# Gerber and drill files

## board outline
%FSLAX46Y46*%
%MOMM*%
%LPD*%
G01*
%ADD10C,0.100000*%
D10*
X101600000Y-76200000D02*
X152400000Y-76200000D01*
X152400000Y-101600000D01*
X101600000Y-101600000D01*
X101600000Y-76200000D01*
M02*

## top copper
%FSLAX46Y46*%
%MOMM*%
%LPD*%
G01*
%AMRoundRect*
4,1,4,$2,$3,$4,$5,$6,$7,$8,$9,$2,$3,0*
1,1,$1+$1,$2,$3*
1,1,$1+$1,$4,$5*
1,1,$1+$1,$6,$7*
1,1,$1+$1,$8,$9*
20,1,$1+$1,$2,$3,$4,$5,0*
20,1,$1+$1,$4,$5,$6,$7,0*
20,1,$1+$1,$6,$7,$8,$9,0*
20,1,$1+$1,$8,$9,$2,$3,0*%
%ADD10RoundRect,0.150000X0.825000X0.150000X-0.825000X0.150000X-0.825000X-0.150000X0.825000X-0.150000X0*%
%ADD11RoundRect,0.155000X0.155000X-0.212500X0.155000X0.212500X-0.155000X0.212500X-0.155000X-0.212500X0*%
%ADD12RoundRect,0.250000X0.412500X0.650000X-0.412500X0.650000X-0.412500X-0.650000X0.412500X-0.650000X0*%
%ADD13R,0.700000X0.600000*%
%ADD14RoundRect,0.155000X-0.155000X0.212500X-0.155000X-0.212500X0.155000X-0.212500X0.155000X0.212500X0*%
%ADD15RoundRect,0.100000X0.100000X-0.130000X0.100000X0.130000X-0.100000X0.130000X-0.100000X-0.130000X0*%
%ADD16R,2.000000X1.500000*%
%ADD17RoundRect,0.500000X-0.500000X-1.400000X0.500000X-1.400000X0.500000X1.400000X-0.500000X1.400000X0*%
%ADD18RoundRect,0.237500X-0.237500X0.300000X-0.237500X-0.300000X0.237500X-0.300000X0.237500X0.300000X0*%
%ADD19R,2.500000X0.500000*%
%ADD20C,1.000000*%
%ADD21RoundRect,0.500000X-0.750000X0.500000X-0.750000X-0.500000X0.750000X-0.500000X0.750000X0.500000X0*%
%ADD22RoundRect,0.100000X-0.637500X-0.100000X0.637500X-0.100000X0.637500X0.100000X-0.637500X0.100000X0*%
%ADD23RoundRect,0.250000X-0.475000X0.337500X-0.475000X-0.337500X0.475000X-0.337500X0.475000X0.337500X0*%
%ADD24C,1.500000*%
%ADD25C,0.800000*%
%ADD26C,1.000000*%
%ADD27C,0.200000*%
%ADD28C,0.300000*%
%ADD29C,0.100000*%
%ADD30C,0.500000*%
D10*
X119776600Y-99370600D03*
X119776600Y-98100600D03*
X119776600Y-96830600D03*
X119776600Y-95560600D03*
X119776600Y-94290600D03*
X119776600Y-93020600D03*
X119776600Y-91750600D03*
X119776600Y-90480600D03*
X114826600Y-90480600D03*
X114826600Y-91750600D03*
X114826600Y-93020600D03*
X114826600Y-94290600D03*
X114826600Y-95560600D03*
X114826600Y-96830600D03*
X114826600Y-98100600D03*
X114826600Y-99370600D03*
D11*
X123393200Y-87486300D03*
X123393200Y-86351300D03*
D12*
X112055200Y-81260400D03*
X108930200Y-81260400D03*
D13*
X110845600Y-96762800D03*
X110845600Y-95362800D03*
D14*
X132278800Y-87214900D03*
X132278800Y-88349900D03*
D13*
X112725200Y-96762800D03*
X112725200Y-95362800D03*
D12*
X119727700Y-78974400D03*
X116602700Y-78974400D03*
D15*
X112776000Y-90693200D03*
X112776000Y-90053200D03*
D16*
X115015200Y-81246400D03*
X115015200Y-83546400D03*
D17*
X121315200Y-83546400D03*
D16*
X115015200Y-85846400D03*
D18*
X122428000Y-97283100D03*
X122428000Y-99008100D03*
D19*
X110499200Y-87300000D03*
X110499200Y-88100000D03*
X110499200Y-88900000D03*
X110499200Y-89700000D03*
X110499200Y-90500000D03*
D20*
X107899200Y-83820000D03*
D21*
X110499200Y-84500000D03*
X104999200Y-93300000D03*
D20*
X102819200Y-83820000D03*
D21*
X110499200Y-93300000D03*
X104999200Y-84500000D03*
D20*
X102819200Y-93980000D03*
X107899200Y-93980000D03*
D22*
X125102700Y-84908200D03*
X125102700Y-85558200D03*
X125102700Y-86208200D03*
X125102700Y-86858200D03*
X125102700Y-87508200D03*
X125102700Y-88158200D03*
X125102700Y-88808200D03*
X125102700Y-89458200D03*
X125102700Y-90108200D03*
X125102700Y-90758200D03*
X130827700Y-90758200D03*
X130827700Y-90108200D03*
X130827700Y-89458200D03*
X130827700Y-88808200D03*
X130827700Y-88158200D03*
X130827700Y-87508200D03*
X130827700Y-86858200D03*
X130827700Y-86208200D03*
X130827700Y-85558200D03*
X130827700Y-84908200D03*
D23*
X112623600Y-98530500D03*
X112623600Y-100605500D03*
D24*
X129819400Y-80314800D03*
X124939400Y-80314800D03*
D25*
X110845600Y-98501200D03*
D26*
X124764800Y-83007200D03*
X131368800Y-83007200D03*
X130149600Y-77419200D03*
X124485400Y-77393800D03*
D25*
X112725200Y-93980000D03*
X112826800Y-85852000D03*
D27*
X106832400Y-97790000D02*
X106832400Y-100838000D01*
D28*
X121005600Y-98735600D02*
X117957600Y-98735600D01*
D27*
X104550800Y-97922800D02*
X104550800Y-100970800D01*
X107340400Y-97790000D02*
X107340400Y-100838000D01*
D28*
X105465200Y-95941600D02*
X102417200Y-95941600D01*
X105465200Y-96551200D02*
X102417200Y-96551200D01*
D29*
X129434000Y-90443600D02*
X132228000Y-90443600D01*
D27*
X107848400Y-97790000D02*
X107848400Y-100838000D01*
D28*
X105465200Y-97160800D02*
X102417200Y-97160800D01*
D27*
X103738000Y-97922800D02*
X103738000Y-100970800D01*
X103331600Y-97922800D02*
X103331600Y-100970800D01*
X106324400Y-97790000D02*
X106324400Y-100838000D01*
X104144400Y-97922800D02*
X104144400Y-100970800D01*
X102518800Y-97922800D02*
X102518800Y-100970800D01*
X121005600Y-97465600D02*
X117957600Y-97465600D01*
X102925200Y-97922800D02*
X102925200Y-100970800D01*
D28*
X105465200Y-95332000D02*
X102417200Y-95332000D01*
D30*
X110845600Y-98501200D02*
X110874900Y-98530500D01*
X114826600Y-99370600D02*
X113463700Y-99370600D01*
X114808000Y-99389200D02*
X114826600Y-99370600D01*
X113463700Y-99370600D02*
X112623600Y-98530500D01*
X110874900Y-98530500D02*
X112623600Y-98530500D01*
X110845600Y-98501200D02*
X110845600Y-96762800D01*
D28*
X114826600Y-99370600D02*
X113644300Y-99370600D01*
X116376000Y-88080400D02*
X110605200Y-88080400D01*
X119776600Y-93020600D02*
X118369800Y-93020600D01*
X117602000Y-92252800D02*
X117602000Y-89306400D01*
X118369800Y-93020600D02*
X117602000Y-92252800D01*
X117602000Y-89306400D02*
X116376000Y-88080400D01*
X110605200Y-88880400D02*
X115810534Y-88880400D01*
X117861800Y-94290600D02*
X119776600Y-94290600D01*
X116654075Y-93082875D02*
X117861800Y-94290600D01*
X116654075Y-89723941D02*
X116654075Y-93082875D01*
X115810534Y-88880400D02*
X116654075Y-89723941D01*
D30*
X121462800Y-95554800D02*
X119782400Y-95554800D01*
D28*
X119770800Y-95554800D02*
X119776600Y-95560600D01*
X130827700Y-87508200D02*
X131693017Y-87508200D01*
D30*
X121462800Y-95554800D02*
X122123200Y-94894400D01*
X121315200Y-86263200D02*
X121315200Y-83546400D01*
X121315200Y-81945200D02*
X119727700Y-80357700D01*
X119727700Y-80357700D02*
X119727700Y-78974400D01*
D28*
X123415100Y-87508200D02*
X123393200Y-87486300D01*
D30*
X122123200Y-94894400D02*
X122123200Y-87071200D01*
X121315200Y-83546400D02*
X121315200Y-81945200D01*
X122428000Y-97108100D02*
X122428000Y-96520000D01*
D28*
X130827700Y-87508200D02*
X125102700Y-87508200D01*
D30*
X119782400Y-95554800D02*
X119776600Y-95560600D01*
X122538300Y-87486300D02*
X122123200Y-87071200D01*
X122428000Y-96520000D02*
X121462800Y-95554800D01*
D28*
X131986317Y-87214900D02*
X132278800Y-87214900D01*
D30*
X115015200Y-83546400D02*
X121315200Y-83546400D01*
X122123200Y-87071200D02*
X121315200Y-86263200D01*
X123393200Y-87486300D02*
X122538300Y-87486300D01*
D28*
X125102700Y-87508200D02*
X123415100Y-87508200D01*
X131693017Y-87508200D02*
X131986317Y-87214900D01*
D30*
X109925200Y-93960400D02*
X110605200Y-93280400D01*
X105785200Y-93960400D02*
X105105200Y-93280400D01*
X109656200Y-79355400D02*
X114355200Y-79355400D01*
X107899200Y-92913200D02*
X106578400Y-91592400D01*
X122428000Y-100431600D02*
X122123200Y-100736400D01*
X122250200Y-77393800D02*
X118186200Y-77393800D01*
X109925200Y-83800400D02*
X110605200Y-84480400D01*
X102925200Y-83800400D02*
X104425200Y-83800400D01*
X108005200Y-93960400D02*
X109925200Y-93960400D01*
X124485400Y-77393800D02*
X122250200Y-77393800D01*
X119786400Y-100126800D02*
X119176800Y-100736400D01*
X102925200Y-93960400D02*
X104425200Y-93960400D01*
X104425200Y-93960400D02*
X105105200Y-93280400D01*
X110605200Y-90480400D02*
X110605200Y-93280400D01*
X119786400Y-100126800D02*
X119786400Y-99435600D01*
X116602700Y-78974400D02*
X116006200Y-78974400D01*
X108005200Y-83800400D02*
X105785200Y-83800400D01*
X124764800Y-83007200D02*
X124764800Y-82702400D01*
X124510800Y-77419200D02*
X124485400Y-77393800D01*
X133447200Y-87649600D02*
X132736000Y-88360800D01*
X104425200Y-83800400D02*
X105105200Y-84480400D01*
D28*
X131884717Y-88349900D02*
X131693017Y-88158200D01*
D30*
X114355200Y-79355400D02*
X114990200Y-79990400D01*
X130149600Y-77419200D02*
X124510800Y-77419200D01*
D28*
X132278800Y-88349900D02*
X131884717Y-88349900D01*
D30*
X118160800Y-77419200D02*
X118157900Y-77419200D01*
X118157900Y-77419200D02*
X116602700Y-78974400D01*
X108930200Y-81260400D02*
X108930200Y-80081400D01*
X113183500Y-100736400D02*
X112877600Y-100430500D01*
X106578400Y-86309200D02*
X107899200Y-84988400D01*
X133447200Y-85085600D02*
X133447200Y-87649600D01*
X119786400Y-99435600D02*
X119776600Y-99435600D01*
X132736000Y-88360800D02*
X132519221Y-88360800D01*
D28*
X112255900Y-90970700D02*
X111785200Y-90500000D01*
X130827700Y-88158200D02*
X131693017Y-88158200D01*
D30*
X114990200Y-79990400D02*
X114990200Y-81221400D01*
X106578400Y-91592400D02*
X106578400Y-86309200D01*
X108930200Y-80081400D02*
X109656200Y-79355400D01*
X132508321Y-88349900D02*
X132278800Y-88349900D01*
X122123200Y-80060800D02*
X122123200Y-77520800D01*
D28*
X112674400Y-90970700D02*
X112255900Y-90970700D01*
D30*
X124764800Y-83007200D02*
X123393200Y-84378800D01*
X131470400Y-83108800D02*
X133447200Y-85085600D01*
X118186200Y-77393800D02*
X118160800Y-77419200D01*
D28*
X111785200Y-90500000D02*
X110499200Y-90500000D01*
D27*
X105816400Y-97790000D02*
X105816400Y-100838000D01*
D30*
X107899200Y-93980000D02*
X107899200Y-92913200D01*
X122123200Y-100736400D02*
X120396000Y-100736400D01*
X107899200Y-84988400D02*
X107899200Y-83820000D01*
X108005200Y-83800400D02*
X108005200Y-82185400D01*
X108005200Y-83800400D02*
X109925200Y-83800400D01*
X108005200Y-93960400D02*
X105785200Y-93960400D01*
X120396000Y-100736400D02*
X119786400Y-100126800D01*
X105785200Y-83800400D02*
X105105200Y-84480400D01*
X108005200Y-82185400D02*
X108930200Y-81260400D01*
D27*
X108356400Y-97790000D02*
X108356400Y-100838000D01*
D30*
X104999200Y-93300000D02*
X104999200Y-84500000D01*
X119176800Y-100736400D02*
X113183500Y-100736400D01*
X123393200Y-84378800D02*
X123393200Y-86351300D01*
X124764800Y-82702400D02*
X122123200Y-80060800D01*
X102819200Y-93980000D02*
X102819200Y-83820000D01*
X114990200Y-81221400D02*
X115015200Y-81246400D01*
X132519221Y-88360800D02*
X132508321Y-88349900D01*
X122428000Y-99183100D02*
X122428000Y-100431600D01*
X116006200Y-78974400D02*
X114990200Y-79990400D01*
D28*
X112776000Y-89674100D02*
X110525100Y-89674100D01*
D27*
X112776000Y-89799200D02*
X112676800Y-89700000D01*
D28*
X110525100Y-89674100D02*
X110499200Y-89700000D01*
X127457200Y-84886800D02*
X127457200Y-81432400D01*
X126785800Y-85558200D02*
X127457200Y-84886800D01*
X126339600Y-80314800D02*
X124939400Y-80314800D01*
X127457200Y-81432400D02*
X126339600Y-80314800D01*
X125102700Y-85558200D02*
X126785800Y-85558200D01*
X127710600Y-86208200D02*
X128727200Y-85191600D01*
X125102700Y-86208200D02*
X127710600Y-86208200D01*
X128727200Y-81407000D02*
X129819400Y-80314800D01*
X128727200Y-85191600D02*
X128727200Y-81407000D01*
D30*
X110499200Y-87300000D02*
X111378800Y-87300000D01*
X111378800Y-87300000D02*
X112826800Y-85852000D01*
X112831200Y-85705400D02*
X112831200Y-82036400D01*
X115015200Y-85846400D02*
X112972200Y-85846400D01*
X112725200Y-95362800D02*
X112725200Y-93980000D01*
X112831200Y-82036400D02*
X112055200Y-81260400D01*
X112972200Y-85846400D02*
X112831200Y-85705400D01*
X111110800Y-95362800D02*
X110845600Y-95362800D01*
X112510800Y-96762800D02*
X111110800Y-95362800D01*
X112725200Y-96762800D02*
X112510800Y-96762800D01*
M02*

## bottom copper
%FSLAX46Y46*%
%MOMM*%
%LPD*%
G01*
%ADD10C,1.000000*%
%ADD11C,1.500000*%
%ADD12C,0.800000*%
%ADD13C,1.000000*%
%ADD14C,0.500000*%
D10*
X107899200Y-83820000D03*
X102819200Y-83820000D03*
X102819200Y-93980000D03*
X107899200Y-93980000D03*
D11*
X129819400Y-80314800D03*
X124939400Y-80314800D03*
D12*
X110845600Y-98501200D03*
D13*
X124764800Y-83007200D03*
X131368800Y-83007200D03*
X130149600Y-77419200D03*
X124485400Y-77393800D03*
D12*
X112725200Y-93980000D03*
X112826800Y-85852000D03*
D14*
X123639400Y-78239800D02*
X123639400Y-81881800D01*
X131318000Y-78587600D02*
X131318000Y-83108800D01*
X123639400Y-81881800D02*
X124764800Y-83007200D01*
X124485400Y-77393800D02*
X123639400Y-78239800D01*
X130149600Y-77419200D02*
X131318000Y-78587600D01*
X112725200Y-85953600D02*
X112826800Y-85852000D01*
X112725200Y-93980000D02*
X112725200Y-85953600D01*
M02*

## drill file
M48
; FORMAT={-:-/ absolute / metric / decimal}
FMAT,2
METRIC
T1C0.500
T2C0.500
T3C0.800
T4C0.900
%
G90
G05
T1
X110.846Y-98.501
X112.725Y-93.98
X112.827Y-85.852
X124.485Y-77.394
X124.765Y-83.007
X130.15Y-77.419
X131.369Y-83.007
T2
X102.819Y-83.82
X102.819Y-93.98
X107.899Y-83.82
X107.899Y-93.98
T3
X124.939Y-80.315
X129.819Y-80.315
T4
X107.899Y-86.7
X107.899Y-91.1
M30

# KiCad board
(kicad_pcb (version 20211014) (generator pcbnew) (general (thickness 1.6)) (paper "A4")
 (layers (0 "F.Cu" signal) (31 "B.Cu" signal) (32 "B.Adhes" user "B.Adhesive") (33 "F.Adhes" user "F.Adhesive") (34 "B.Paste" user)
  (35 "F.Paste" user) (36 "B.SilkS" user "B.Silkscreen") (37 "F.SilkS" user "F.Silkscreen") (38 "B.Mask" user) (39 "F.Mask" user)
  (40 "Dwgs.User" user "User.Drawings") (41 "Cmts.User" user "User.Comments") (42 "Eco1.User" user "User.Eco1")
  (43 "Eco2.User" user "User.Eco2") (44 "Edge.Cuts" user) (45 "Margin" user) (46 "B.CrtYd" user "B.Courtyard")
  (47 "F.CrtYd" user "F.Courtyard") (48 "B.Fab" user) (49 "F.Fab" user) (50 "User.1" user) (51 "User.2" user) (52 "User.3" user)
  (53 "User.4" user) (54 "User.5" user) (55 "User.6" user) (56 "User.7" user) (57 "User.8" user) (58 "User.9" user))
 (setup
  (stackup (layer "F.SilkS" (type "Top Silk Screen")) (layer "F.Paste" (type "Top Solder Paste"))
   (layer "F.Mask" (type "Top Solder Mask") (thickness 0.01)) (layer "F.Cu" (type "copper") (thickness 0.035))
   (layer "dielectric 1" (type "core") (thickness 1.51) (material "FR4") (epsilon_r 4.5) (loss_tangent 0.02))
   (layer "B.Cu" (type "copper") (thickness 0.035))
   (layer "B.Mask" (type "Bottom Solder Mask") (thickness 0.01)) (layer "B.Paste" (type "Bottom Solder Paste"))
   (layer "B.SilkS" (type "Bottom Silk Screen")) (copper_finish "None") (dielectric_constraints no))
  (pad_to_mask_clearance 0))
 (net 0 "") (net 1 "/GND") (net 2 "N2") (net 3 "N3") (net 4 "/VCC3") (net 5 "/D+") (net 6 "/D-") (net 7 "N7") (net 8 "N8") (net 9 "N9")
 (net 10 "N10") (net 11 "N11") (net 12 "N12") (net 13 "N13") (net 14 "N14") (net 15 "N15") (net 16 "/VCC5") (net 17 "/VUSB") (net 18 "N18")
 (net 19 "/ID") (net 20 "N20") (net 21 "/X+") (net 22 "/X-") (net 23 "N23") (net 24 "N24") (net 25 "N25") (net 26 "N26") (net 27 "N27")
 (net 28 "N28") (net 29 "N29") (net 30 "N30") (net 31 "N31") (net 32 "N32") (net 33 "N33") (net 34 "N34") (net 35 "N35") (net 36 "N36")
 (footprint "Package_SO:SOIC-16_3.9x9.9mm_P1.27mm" (layer "F.Cu") (at 117.3016 94.9256 180) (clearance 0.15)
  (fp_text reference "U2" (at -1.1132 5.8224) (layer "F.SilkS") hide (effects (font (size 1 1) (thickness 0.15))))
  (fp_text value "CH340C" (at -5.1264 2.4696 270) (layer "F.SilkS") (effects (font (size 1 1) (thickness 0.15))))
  (pad "1" smd roundrect (at -2.475 -4.445 180) (size 1.95 0.6) (layers "F.Cu" "F.Paste" "F.Mask") (roundrect_rratio 0.25) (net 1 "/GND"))
  (pad "2" smd roundrect (at -2.475 -3.175 180) (size 1.95 0.6) (layers "F.Cu" "F.Paste" "F.Mask") (roundrect_rratio 0.25) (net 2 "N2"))
  (pad "3" smd roundrect (at -2.475 -1.905 180) (size 1.95 0.6) (layers "F.Cu" "F.Paste" "F.Mask") (roundrect_rratio 0.25) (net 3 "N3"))
  (pad "4" smd roundrect (at -2.475 -0.635 180) (size 1.95 0.6) (layers "F.Cu" "F.Paste" "F.Mask") (roundrect_rratio 0.25) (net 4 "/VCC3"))
  (pad "5" smd roundrect (at -2.475 0.635 180) (size 1.95 0.6) (layers "F.Cu" "F.Paste" "F.Mask") (roundrect_rratio 0.25) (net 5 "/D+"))
  (pad "6" smd roundrect (at -2.475 1.905 180) (size 1.95 0.6) (layers "F.Cu" "F.Paste" "F.Mask") (roundrect_rratio 0.25) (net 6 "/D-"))
  (pad "7" smd roundrect (at -2.475 3.175 180) (size 1.95 0.6) (layers "F.Cu" "F.Paste" "F.Mask") (roundrect_rratio 0.25) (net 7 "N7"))
  (pad "8" smd roundrect (at -2.475 4.445 180) (size 1.95 0.6) (layers "F.Cu" "F.Paste" "F.Mask") (roundrect_rratio 0.25) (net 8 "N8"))
  (pad "9" smd roundrect (at 2.475 4.445 180) (size 1.95 0.6) (layers "F.Cu" "F.Paste" "F.Mask") (roundrect_rratio 0.25) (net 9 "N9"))
  (pad "10" smd roundrect (at 2.475 3.175 180) (size 1.95 0.6) (layers "F.Cu" "F.Paste" "F.Mask") (roundrect_rratio 0.25) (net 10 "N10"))
  (pad "11" smd roundrect (at 2.475 1.905 180) (size 1.95 0.6) (layers "F.Cu" "F.Paste" "F.Mask") (roundrect_rratio 0.25) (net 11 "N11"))
  (pad "12" smd roundrect (at 2.475 0.635 180) (size 1.95 0.6) (layers "F.Cu" "F.Paste" "F.Mask") (roundrect_rratio 0.25) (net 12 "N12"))
  (pad "13" smd roundrect (at 2.475 -0.635 180) (size 1.95 0.6) (layers "F.Cu" "F.Paste" "F.Mask") (roundrect_rratio 0.25) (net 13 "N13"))
  (pad "14" smd roundrect (at 2.475 -1.905 180) (size 1.95 0.6) (layers "F.Cu" "F.Paste" "F.Mask") (roundrect_rratio 0.25) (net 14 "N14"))
  (pad "15" smd roundrect (at 2.475 -3.175 180) (size 1.95 0.6) (layers "F.Cu" "F.Paste" "F.Mask") (roundrect_rratio 0.25) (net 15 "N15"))
  (pad "16" smd roundrect (at 2.475 -4.445 180) (size 1.95 0.6) (layers "F.Cu" "F.Paste" "F.Mask") (roundrect_rratio 0.25) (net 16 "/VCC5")))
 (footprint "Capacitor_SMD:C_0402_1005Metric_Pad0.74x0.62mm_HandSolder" (layer "F.Cu") (at 123.3932 86.9188 90)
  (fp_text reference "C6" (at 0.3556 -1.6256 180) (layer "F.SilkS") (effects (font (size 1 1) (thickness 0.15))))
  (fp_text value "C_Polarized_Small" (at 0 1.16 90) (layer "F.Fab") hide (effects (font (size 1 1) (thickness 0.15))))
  (pad "1" smd roundrect (at -0.5675 0 90) (size 0.735 0.62) (layers "F.Cu" "F.Paste" "F.Mask") (roundrect_rratio 0.25) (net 4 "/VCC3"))
  (pad "2" smd roundrect (at 0.5675 0 90) (size 0.735 0.62) (layers "F.Cu" "F.Paste" "F.Mask") (roundrect_rratio 0.25) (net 1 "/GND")))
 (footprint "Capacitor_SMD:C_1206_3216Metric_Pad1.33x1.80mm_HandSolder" (layer "F.Cu") (at 110.4927 81.2604 180)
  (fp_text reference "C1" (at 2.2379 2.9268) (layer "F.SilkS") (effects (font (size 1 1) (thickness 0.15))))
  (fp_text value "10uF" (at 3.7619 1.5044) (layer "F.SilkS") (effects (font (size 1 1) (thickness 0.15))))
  (pad "1" smd roundrect (at -1.5625 0 180) (size 1.325 1.8) (layers "F.Cu" "F.Paste" "F.Mask") (roundrect_rratio 0.188679) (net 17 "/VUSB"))
  (pad "2" smd roundrect (at 1.5625 0 180) (size 1.325 1.8) (layers "F.Cu" "F.Paste" "F.Mask") (roundrect_rratio 0.188679) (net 1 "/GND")))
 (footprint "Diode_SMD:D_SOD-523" (layer "F.Cu") (at 110.8456 96.0628 90)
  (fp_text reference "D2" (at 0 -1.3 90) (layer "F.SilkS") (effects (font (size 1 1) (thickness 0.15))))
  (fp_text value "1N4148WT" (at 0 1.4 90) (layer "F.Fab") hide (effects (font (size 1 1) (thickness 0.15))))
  (pad "1" smd rect (at -0.7 0 270) (size 0.6 0.7) (layers "F.Cu" "F.Paste" "F.Mask") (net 16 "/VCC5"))
  (pad "2" smd rect (at 0.7 0 270) (size 0.6 0.7) (layers "F.Cu" "F.Paste" "F.Mask") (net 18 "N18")))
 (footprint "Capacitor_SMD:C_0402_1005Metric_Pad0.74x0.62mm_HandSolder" (layer "F.Cu") (at 132.2788 87.7824 -90)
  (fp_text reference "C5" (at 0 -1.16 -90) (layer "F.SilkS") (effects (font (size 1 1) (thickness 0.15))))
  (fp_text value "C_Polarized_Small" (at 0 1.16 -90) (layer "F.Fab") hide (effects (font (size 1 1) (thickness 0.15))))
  (pad "1" smd roundrect (at -0.5675 0 270) (size 0.735 0.62) (layers "F.Cu" "F.Paste" "F.Mask") (roundrect_rratio 0.25) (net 4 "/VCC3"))
  (pad "2" smd roundrect (at 0.5675 0 270) (size 0.735 0.62) (layers "F.Cu" "F.Paste" "F.Mask") (roundrect_rratio 0.25) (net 1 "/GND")))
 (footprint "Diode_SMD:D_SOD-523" (layer "F.Cu") (at 112.7252 96.0628 90)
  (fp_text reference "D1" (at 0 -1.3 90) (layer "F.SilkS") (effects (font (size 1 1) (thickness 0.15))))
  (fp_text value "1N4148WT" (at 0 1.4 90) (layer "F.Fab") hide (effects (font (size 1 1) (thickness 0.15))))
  (pad "1" smd rect (at -0.7 0 270) (size 0.6 0.7) (layers "F.Cu" "F.Paste" "F.Mask") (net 18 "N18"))
  (pad "2" smd rect (at 0.7 0 270) (size 0.6 0.7) (layers "F.Cu" "F.Paste" "F.Mask") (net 17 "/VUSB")))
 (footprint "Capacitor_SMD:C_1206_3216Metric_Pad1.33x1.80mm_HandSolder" (layer "F.Cu") (at 118.1652 78.9744 180)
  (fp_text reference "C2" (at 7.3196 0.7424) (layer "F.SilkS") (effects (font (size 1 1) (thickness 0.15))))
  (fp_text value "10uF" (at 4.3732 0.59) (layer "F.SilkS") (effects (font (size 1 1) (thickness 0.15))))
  (pad "1" smd roundrect (at -1.5625 0 180) (size 1.325 1.8) (layers "F.Cu" "F.Paste" "F.Mask") (roundrect_rratio 0.188679) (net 4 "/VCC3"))
  (pad "2" smd roundrect (at 1.5625 0 180) (size 1.325 1.8) (layers "F.Cu" "F.Paste" "F.Mask") (roundrect_rratio 0.188679) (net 1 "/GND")))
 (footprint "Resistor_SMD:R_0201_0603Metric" (layer "F.Cu") (at 112.776 90.3732 90)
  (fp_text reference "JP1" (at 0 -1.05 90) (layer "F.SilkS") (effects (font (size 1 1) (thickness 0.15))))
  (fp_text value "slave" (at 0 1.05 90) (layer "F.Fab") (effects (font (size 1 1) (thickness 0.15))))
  (pad "" smd roundrect (at -0.345 0 90) (size 0.318 0.36) (layers "F.Paste") (roundrect_rratio 0.25))
  (pad "" smd roundrect (at 0.345 0 90) (size 0.318 0.36) (layers "F.Paste") (roundrect_rratio 0.25))
  (pad "1" smd roundrect (at -0.32 0 90) (size 0.46 0.4) (layers "F.Cu" "F.Mask") (roundrect_rratio 0.25) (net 1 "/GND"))
  (pad "2" smd roundrect (at 0.32 0 90) (size 0.46 0.4) (layers "F.Cu" "F.Mask") (roundrect_rratio 0.25) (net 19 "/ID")))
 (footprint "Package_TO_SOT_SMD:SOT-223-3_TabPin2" (layer "F.Cu") (at 118.1652 83.5464)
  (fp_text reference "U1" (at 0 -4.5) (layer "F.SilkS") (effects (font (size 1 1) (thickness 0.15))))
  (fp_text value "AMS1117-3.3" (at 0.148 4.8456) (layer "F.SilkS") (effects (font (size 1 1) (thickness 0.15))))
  (pad "1" smd rect (at -3.15 -2.3) (size 2 1.5) (layers "F.Cu" "F.Paste" "F.Mask") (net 1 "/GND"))
  (pad "2" smd rect (at -3.15 0) (size 2 1.5) (layers "F.Cu" "F.Paste" "F.Mask") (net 4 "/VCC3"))
  (pad "2" smd roundrect (at 3.15 0) (size 2 3.8) (layers "F.Cu" "F.Paste" "F.Mask") (roundrect_rratio 0.25) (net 4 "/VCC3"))
  (pad "3" smd rect (at -3.15 2.3) (size 2 1.5) (layers "F.Cu" "F.Paste" "F.Mask") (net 17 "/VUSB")))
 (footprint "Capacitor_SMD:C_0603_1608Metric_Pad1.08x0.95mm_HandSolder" (layer "F.Cu") (at 122.428 98.1456 -90)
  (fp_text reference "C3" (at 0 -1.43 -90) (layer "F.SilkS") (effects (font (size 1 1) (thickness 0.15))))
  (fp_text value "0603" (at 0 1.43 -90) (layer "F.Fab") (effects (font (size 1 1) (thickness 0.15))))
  (pad "1" smd roundrect (at -0.8625 0 270) (size 1.075 0.95) (layers "F.Cu" "F.Paste" "F.Mask") (roundrect_rratio 0.25) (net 4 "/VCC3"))
  (pad "2" smd roundrect (at 0.8625 0 270) (size 1.075 0.95) (layers "F.Cu" "F.Paste" "F.Mask") (roundrect_rratio 0.25) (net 1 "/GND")))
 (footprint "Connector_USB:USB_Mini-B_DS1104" (layer "F.Cu") (at 107.8992 88.9 -90)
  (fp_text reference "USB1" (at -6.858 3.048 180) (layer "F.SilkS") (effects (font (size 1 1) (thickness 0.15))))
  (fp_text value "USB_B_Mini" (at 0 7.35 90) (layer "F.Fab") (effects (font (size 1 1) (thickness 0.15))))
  (pad "" np_thru_hole circle (at 2.2 0 270) (size 0.9 0.9) (drill 0.9) (layers *.Cu *.Mask))
  (pad "" np_thru_hole circle (at -2.2 0 270) (size 0.9 0.9) (drill 0.9) (layers *.Cu *.Mask))
  (pad "1" smd rect (at -1.6 -2.6 270) (size 0.5 2.5) (layers "F.Cu" "F.Paste" "F.Mask") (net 17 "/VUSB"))
  (pad "2" smd rect (at -0.8 -2.6 270) (size 0.5 2.5) (layers "F.Cu" "F.Paste" "F.Mask") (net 6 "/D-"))
  (pad "3" smd rect (at 0 -2.6 270) (size 0.5 2.5) (layers "F.Cu" "F.Paste" "F.Mask") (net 5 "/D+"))
  (pad "4" smd rect (at 0.8 -2.6 270) (size 0.5 2.5) (layers "F.Cu" "F.Paste" "F.Mask") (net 19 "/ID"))
  (pad "5" smd rect (at 1.6 -2.6 270) (size 0.5 2.5) (layers "F.Cu" "F.Paste" "F.Mask") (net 1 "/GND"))
  (pad "6" thru_hole circle (at -5.08 0 270) (size 1 1) (drill 0.5) (layers *.Cu *.Mask) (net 1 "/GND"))
  (pad "6" smd roundrect (at -4.4 -2.6 270) (size 2 2.5) (layers "F.Cu" "F.Paste" "F.Mask") (roundrect_rratio 0.25) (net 1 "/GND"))
  (pad "6" smd roundrect (at 4.4 2.9 270) (size 2 2.5) (layers "F.Cu" "F.Paste" "F.Mask") (roundrect_rratio 0.25) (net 1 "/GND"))
  (pad "6" thru_hole circle (at -5.08 5.08 270) (size 1 1) (drill 0.5) (layers *.Cu *.Mask) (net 1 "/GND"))
  (pad "6" smd roundrect (at 4.4 -2.6 270) (size 2 2.5) (layers "F.Cu" "F.Paste" "F.Mask") (roundrect_rratio 0.25) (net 1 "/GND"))
  (pad "6" smd roundrect (at -4.4 2.9 270) (size 2 2.5) (layers "F.Cu" "F.Paste" "F.Mask") (roundrect_rratio 0.25) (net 1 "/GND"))
  (pad "6" thru_hole circle (at 5.08 5.08 270) (size 1 1) (drill 0.5) (layers *.Cu *.Mask) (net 1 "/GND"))
  (pad "6" thru_hole circle (at 5.08 0 270) (size 1 1) (drill 0.5) (layers *.Cu *.Mask) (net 1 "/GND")))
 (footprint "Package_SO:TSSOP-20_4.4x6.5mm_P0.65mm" (layer "F.Cu") (at 127.9652 87.8332)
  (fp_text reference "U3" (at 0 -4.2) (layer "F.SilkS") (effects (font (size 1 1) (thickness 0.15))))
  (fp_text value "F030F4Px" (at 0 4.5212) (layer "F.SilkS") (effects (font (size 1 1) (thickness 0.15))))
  (pad "1" smd roundrect (at -2.8625 -2.925) (size 1.475 0.4) (layers "F.Cu" "F.Paste" "F.Mask") (roundrect_rratio 0.25) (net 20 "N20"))
  (pad "2" smd roundrect (at -2.8625 -2.275) (size 1.475 0.4) (layers "F.Cu" "F.Paste" "F.Mask") (roundrect_rratio 0.25) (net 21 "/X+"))
  (pad "3" smd roundrect (at -2.8625 -1.625) (size 1.475 0.4) (layers "F.Cu" "F.Paste" "F.Mask") (roundrect_rratio 0.25) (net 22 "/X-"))
  (pad "4" smd roundrect (at -2.8625 -0.975) (size 1.475 0.4) (layers "F.Cu" "F.Paste" "F.Mask") (roundrect_rratio 0.25) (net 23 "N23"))
  (pad "5" smd roundrect (at -2.8625 -0.325) (size 1.475 0.4) (layers "F.Cu" "F.Paste" "F.Mask") (roundrect_rratio 0.25) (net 4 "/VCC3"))
  (pad "6" smd roundrect (at -2.8625 0.325) (size 1.475 0.4) (layers "F.Cu" "F.Paste" "F.Mask") (roundrect_rratio 0.25) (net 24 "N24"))
  (pad "7" smd roundrect (at -2.8625 0.975) (size 1.475 0.4) (layers "F.Cu" "F.Paste" "F.Mask") (roundrect_rratio 0.25) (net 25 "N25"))
  (pad "8" smd roundrect (at -2.8625 1.625) (size 1.475 0.4) (layers "F.Cu" "F.Paste" "F.Mask") (roundrect_rratio 0.25) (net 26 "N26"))
  (pad "9" smd roundrect (at -2.8625 2.275) (size 1.475 0.4) (layers "F.Cu" "F.Paste" "F.Mask") (roundrect_rratio 0.25) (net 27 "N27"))
  (pad "10" smd roundrect (at -2.8625 2.925) (size 1.475 0.4) (layers "F.Cu" "F.Paste" "F.Mask") (roundrect_rratio 0.25) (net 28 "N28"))
  (pad "11" smd roundrect (at 2.8625 2.925) (size 1.475 0.4) (layers "F.Cu" "F.Paste" "F.Mask") (roundrect_rratio 0.25) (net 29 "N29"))
  (pad "12" smd roundrect (at 2.8625 2.275) (size 1.475 0.4) (layers "F.Cu" "F.Paste" "F.Mask") (roundrect_rratio 0.25) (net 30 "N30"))
  (pad "13" smd roundrect (at 2.8625 1.625) (size 1.475 0.4) (layers "F.Cu" "F.Paste" "F.Mask") (roundrect_rratio 0.25) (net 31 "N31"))
  (pad "14" smd roundrect (at 2.8625 0.975) (size 1.475 0.4) (layers "F.Cu" "F.Paste" "F.Mask") (roundrect_rratio 0.25) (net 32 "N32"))
  (pad "15" smd roundrect (at 2.8625 0.325) (size 1.475 0.4) (layers "F.Cu" "F.Paste" "F.Mask") (roundrect_rratio 0.25) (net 1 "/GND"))
  (pad "16" smd roundrect (at 2.8625 -0.325) (size 1.475 0.4) (layers "F.Cu" "F.Paste" "F.Mask") (roundrect_rratio 0.25) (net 4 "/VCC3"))
  (pad "17" smd roundrect (at 2.8625 -0.975) (size 1.475 0.4) (layers "F.Cu" "F.Paste" "F.Mask") (roundrect_rratio 0.25) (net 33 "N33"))
  (pad "18" smd roundrect (at 2.8625 -1.625) (size 1.475 0.4) (layers "F.Cu" "F.Paste" "F.Mask") (roundrect_rratio 0.25) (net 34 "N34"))
  (pad "19" smd roundrect (at 2.8625 -2.275) (size 1.475 0.4) (layers "F.Cu" "F.Paste" "F.Mask") (roundrect_rratio 0.25) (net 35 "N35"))
  (pad "20" smd roundrect (at 2.8625 -2.925) (size 1.475 0.4) (layers "F.Cu" "F.Paste" "F.Mask") (roundrect_rratio 0.25) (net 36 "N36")))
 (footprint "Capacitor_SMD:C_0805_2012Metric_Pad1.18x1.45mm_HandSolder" (layer "F.Cu") (at 112.6236 99.568 -90)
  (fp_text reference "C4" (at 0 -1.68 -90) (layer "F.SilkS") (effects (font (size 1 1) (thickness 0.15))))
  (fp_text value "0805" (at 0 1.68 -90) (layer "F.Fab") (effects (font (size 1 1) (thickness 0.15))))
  (pad "1" smd roundrect (at -1.0375 0 270) (size 1.175 1.45) (layers "F.Cu" "F.Paste" "F.Mask") (roundrect_rratio 0.212766)
   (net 16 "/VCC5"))
  (pad "2" smd roundrect (at 1.0375 0 270) (size 1.175 1.45) (layers "F.Cu" "F.Paste" "F.Mask") (roundrect_rratio 0.212766) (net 1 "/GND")))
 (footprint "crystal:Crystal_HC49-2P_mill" (layer "B.Cu") (at 129.8194 80.3148 180)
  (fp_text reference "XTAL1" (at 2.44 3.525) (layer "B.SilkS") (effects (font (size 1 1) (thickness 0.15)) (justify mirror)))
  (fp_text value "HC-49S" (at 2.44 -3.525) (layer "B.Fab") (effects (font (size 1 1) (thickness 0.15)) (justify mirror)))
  (pad "1" thru_hole circle (at 0 0 180) (size 1.5 1.5) (drill 0.8) (layers *.Cu *.Mask) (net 22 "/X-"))
  (pad "2" thru_hole circle (at 4.88 0 180) (size 1.5 1.5) (drill 0.8) (layers *.Cu *.Mask) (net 21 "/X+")))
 (gr_rect (start 101.6 76.2) (end 152.4 101.6) (layer "Edge.Cuts") (width 0.1) (fill none))
 (segment (start 106.8324 97.79) (end 106.8324 100.838) (width 0.2) (layer "F.Cu") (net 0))
 (segment (start 121.0056 98.7356) (end 117.9576 98.7356) (width 0.3) (layer "F.Cu") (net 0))
 (segment (start 104.5508 97.9228) (end 104.5508 100.9708) (width 0.2) (layer "F.Cu") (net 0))
 (segment (start 107.3404 97.79) (end 107.3404 100.838) (width 0.2) (layer "F.Cu") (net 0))
 (segment (start 105.4652 95.9416) (end 102.4172 95.9416) (width 0.3) (layer "F.Cu") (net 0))
 (segment (start 105.4652 96.5512) (end 102.4172 96.5512) (width 0.3) (layer "F.Cu") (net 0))
 (segment (start 129.434 90.4436) (end 132.228 90.4436) (width 0.1) (layer "F.Cu") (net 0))
 (segment (start 107.8484 97.79) (end 107.8484 100.838) (width 0.2) (layer "F.Cu") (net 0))
 (segment (start 105.4652 97.1608) (end 102.4172 97.1608) (width 0.3) (layer "F.Cu") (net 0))
 (segment (start 103.738 97.9228) (end 103.738 100.9708) (width 0.2) (layer "F.Cu") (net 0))
 (segment (start 103.3316 97.9228) (end 103.3316 100.9708) (width 0.2) (layer "F.Cu") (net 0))
 (segment (start 106.3244 97.79) (end 106.3244 100.838) (width 0.2) (layer "F.Cu") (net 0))
 (segment (start 104.1444 97.9228) (end 104.1444 100.9708) (width 0.2) (layer "F.Cu") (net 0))
 (segment (start 102.5188 97.9228) (end 102.5188 100.9708) (width 0.2) (layer "F.Cu") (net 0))
 (segment (start 121.0056 97.4656) (end 117.9576 97.4656) (width 0.2) (layer "F.Cu") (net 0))
 (segment (start 102.9252 97.9228) (end 102.9252 100.9708) (width 0.2) (layer "F.Cu") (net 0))
 (segment (start 105.4652 95.332) (end 102.4172 95.332) (width 0.3) (layer "F.Cu") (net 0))
 (segment (start 110.8456 98.5012) (end 110.8749 98.5305) (width 0.5) (layer "F.Cu") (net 16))
 (segment (start 114.8266 99.3706) (end 113.4637 99.3706) (width 0.5) (layer "F.Cu") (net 16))
 (segment (start 114.808 99.3892) (end 114.8266 99.3706) (width 0.5) (layer "F.Cu") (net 16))
 (segment (start 113.4637 99.3706) (end 112.6236 98.5305) (width 0.5) (layer "F.Cu") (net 16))
 (segment (start 110.8749 98.5305) (end 112.6236 98.5305) (width 0.5) (layer "F.Cu") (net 16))
 (segment (start 110.8456 98.5012) (end 110.8456 96.7628) (width 0.5) (layer "F.Cu") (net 16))
 (segment (start 114.8266 99.3706) (end 113.6443 99.3706) (width 0.3) (layer "F.Cu") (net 16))
 (via (at 110.8456 98.5012) (size 0.8) (drill 0.5) (layers "F.Cu" "B.Cu") (free) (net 16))
 (segment (start 116.376 88.0804) (end 110.6052 88.0804) (width 0.3) (layer "F.Cu") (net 6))
 (segment (start 119.7766 93.0206) (end 118.3698 93.0206) (width 0.3) (layer "F.Cu") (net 6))
 (segment (start 117.602 92.2528) (end 117.602 89.3064) (width 0.3) (layer "F.Cu") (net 6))
 (segment (start 118.3698 93.0206) (end 117.602 92.2528) (width 0.3) (layer "F.Cu") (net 6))
 (segment (start 117.602 89.3064) (end 116.376 88.0804) (width 0.3) (layer "F.Cu") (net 6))
 (segment (start 110.6052 88.8804) (end 115.810534 88.8804) (width 0.3) (layer "F.Cu") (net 5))
 (segment (start 117.8618 94.2906) (end 119.7766 94.2906) (width 0.3) (layer "F.Cu") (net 5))
 (segment (start 116.654075 93.082875) (end 117.8618 94.2906) (width 0.3) (layer "F.Cu") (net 5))
 (segment (start 116.654075 89.723941) (end 116.654075 93.082875) (width 0.3) (layer "F.Cu") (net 5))
 (segment (start 115.810534 88.8804) (end 116.654075 89.723941) (width 0.3) (layer "F.Cu") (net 5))
 (segment (start 121.4628 95.5548) (end 119.7824 95.5548) (width 0.5) (layer "F.Cu") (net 4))
 (segment (start 119.7708 95.5548) (end 119.7766 95.5606) (width 0.3) (layer "F.Cu") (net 4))
 (segment (start 130.8277 87.5082) (end 131.693017 87.5082) (width 0.3) (layer "F.Cu") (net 4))
 (segment (start 121.4628 95.5548) (end 122.1232 94.8944) (width 0.5) (layer "F.Cu") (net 4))
 (segment (start 121.3152 86.2632) (end 121.3152 83.5464) (width 0.5) (layer "F.Cu") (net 4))
 (segment (start 121.3152 81.9452) (end 119.7277 80.3577) (width 0.5) (layer "F.Cu") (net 4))
 (segment (start 119.7277 80.3577) (end 119.7277 78.9744) (width 0.5) (layer "F.Cu") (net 4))
 (segment (start 123.4151 87.5082) (end 123.3932 87.4863) (width 0.3) (layer "F.Cu") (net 4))
 (segment (start 122.1232 94.8944) (end 122.1232 87.0712) (width 0.5) (layer "F.Cu") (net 4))
 (segment (start 121.3152 83.5464) (end 121.3152 81.9452) (width 0.5) (layer "F.Cu") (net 4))
 (segment (start 122.428 97.1081) (end 122.428 96.52) (width 0.5) (layer "F.Cu") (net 4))
 (segment (start 130.8277 87.5082) (end 125.1027 87.5082) (width 0.3) (layer "F.Cu") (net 4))
 (segment (start 119.7824 95.5548) (end 119.7766 95.5606) (width 0.5) (layer "F.Cu") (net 4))
 (segment (start 122.5383 87.4863) (end 122.1232 87.0712) (width 0.5) (layer "F.Cu") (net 4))
 (segment (start 122.428 96.52) (end 121.4628 95.5548) (width 0.5) (layer "F.Cu") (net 4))
 (segment (start 131.986317 87.2149) (end 132.2788 87.2149) (width 0.3) (layer "F.Cu") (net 4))
 (segment (start 115.0152 83.5464) (end 121.3152 83.5464) (width 0.5) (layer "F.Cu") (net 4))
 (segment (start 122.1232 87.0712) (end 121.3152 86.2632) (width 0.5) (layer "F.Cu") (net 4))
 (segment (start 123.3932 87.4863) (end 122.5383 87.4863) (width 0.5) (layer "F.Cu") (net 4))
 (segment (start 125.1027 87.5082) (end 123.4151 87.5082) (width 0.3) (layer "F.Cu") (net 4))
 (segment (start 131.693017 87.5082) (end 131.986317 87.2149) (width 0.3) (layer "F.Cu") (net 4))
 (segment (start 109.9252 93.9604) (end 110.6052 93.2804) (width 0.5) (layer "F.Cu") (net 1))
 (segment (start 105.7852 93.9604) (end 105.1052 93.2804) (width 0.5) (layer "F.Cu") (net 1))
 (segment (start 109.6562 79.3554) (end 114.3552 79.3554) (width 0.5) (layer "F.Cu") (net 1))
 (segment (start 107.8992 92.9132) (end 106.5784 91.5924) (width 0.5) (layer "F.Cu") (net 1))
 (segment (start 122.428 100.4316) (end 122.1232 100.7364) (width 0.5) (layer "F.Cu") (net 1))
 (segment (start 122.2502 77.3938) (end 118.1862 77.3938) (width 0.5) (layer "F.Cu") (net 1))
 (segment (start 109.9252 83.8004) (end 110.6052 84.4804) (width 0.5) (layer "F.Cu") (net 1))
 (segment (start 102.9252 83.8004) (end 104.4252 83.8004) (width 0.5) (layer "F.Cu") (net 1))
 (segment (start 108.0052 93.9604) (end 109.9252 93.9604) (width 0.5) (layer "F.Cu") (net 1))
 (segment (start 124.4854 77.3938) (end 122.2502 77.3938) (width 0.5) (layer "F.Cu") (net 1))
 (segment (start 119.7864 100.1268) (end 119.1768 100.7364) (width 0.5) (layer "F.Cu") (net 1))
 (segment (start 102.9252 93.9604) (end 104.4252 93.9604) (width 0.5) (layer "F.Cu") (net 1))
 (segment (start 104.4252 93.9604) (end 105.1052 93.2804) (width 0.5) (layer "F.Cu") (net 1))
 (segment (start 110.6052 90.4804) (end 110.6052 93.2804) (width 0.5) (layer "F.Cu") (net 1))
 (segment (start 119.7864 100.1268) (end 119.7864 99.4356) (width 0.5) (layer "F.Cu") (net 1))
 (segment (start 116.6027 78.9744) (end 116.0062 78.9744) (width 0.5) (layer "F.Cu") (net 1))
 (segment (start 108.0052 83.8004) (end 105.7852 83.8004) (width 0.5) (layer "F.Cu") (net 1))
 (segment (start 124.7648 83.0072) (end 124.7648 82.7024) (width 0.5) (layer "F.Cu") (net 1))
 (segment (start 124.5108 77.4192) (end 124.4854 77.3938) (width 0.5) (layer "F.Cu") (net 1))
 (segment (start 133.4472 87.6496) (end 132.736 88.3608) (width 0.5) (layer "F.Cu") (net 1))
 (segment (start 104.4252 83.8004) (end 105.1052 84.4804) (width 0.5) (layer "F.Cu") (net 1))
 (segment (start 131.884717 88.3499) (end 131.693017 88.1582) (width 0.3) (layer "F.Cu") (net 1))
 (segment (start 114.3552 79.3554) (end 114.9902 79.9904) (width 0.5) (layer "F.Cu") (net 1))
 (segment (start 130.1496 77.4192) (end 124.5108 77.4192) (width 0.5) (layer "F.Cu") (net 1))
 (segment (start 132.2788 88.3499) (end 131.884717 88.3499) (width 0.3) (layer "F.Cu") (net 1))
 (segment (start 118.1608 77.4192) (end 118.1579 77.4192) (width 0.5) (layer "F.Cu") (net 1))
 (segment (start 118.1579 77.4192) (end 116.6027 78.9744) (width 0.5) (layer "F.Cu") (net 1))
 (segment (start 108.9302 81.2604) (end 108.9302 80.0814) (width 0.5) (layer "F.Cu") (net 1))
 (segment (start 113.1835 100.7364) (end 112.8776 100.4305) (width 0.5) (layer "F.Cu") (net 1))
 (segment (start 106.5784 86.3092) (end 107.8992 84.9884) (width 0.5) (layer "F.Cu") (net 1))
 (segment (start 133.4472 85.0856) (end 133.4472 87.6496) (width 0.5) (layer "F.Cu") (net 1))
 (segment (start 119.7864 99.4356) (end 119.7766 99.4356) (width 0.5) (layer "F.Cu") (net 1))
 (segment (start 132.736 88.3608) (end 132.519221 88.3608) (width 0.5) (layer "F.Cu") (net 1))
 (segment (start 112.2559 90.9707) (end 111.7852 90.5) (width 0.3) (layer "F.Cu") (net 1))
 (segment (start 130.8277 88.1582) (end 131.693017 88.1582) (width 0.3) (layer "F.Cu") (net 1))
 (segment (start 114.9902 79.9904) (end 114.9902 81.2214) (width 0.5) (layer "F.Cu") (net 1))
 (segment (start 106.5784 91.5924) (end 106.5784 86.3092) (width 0.5) (layer "F.Cu") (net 1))
 (segment (start 108.9302 80.0814) (end 109.6562 79.3554) (width 0.5) (layer "F.Cu") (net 1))
 (segment (start 132.508321 88.3499) (end 132.2788 88.3499) (width 0.5) (layer "F.Cu") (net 1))
 (segment (start 122.1232 80.0608) (end 122.1232 77.5208) (width 0.5) (layer "F.Cu") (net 1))
 (segment (start 112.6744 90.9707) (end 112.2559 90.9707) (width 0.3) (layer "F.Cu") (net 1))
 (segment (start 124.7648 83.0072) (end 123.3932 84.3788) (width 0.5) (layer "F.Cu") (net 1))
 (segment (start 131.4704 83.1088) (end 133.4472 85.0856) (width 0.5) (layer "F.Cu") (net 1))
 (segment (start 118.1862 77.3938) (end 118.1608 77.4192) (width 0.5) (layer "F.Cu") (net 1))
 (segment (start 111.7852 90.5) (end 110.4992 90.5) (width 0.3) (layer "F.Cu") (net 1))
 (segment (start 105.8164 97.79) (end 105.8164 100.838) (width 0.2) (layer "F.Cu") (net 1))
 (segment (start 107.8992 93.98) (end 107.8992 92.9132) (width 0.5) (layer "F.Cu") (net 1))
 (segment (start 122.1232 100.7364) (end 120.396 100.7364) (width 0.5) (layer "F.Cu") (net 1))
 (segment (start 107.8992 84.9884) (end 107.8992 83.82) (width 0.5) (layer "F.Cu") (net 1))
 (segment (start 108.0052 83.8004) (end 108.0052 82.1854) (width 0.5) (layer "F.Cu") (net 1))
 (segment (start 108.0052 83.8004) (end 109.9252 83.8004) (width 0.5) (layer "F.Cu") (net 1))
 (segment (start 108.0052 93.9604) (end 105.7852 93.9604) (width 0.5) (layer "F.Cu") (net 1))
 (segment (start 120.396 100.7364) (end 119.7864 100.1268) (width 0.5) (layer "F.Cu") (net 1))
 (segment (start 105.7852 83.8004) (end 105.1052 84.4804) (width 0.5) (layer "F.Cu") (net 1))
 (segment (start 108.0052 82.1854) (end 108.9302 81.2604) (width 0.5) (layer "F.Cu") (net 1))
 (segment (start 108.3564 97.79) (end 108.3564 100.838) (width 0.2) (layer "F.Cu") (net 1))
 (segment (start 104.9992 93.3) (end 104.9992 84.5) (width 0.5) (layer "F.Cu") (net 1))
 (segment (start 119.1768 100.7364) (end 113.1835 100.7364) (width 0.5) (layer "F.Cu") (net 1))
 (segment (start 123.3932 84.3788) (end 123.3932 86.3513) (width 0.5) (layer "F.Cu") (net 1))
 (segment (start 124.7648 82.7024) (end 122.1232 80.0608) (width 0.5) (layer "F.Cu") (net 1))
 (segment (start 102.8192 93.98) (end 102.8192 83.82) (width 0.5) (layer "F.Cu") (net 1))
 (segment (start 114.9902 81.2214) (end 115.0152 81.2464) (width 0.5) (layer "F.Cu") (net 1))
 (segment (start 132.519221 88.3608) (end 132.508321 88.3499) (width 0.5) (layer "F.Cu") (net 1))
 (segment (start 122.428 99.1831) (end 122.428 100.4316) (width 0.5) (layer "F.Cu") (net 1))
 (segment (start 116.0062 78.9744) (end 114.9902 79.9904) (width 0.5) (layer "F.Cu") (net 1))
 (via (at 124.7648 83.0072) (size 1) (drill 0.5) (layers "F.Cu" "B.Cu") (free) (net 1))
 (via (at 131.3688 83.0072) (size 1) (drill 0.5) (layers "F.Cu" "B.Cu") (free) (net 1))
 (via (at 130.1496 77.4192) (size 1) (drill 0.5) (layers "F.Cu" "B.Cu") (free) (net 1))
 (via (at 124.4854 77.3938) (size 1) (drill 0.5) (layers "F.Cu" "B.Cu") (free) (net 1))
 (segment (start 123.6394 78.2398) (end 123.6394 81.8818) (width 0.5) (layer "B.Cu") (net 1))
 (segment (start 131.318 78.5876) (end 131.318 83.1088) (width 0.5) (layer "B.Cu") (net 1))
 (segment (start 123.6394 81.8818) (end 124.7648 83.0072) (width 0.5) (layer "B.Cu") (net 1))
 (segment (start 124.4854 77.3938) (end 123.6394 78.2398) (width 0.5) (layer "B.Cu") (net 1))
 (segment (start 130.1496 77.4192) (end 131.318 78.5876) (width 0.5) (layer "B.Cu") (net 1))
 (segment (start 112.776 89.6741) (end 110.5251 89.6741) (width 0.3) (layer "F.Cu") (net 19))
 (segment (start 112.776 89.7992) (end 112.6768 89.7) (width 0.2) (layer "F.Cu") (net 19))
 (segment (start 110.5251 89.6741) (end 110.4992 89.7) (width 0.3) (layer "F.Cu") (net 19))
 (segment (start 127.4572 84.8868) (end 127.4572 81.4324) (width 0.3) (layer "F.Cu") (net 21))
 (segment (start 126.7858 85.5582) (end 127.4572 84.8868) (width 0.3) (layer "F.Cu") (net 21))
 (segment (start 126.3396 80.3148) (end 124.9394 80.3148) (width 0.3) (layer "F.Cu") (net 21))
 (segment (start 127.4572 81.4324) (end 126.3396 80.3148) (width 0.3) (layer "F.Cu") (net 21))
 (segment (start 125.1027 85.5582) (end 126.7858 85.5582) (width 0.3) (layer "F.Cu") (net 21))
 (segment (start 127.7106 86.2082) (end 128.7272 85.1916) (width 0.3) (layer "F.Cu") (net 22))
 (segment (start 125.1027 86.2082) (end 127.7106 86.2082) (width 0.3) (layer "F.Cu") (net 22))
 (segment (start 128.7272 81.407) (end 129.8194 80.3148) (width 0.3) (layer "F.Cu") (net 22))
 (segment (start 128.7272 85.1916) (end 128.7272 81.407) (width 0.3) (layer "F.Cu") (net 22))
 (segment (start 110.4992 87.3) (end 111.3788 87.3) (width 0.5) (layer "F.Cu") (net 17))
 (segment (start 111.3788 87.3) (end 112.8268 85.852) (width 0.5) (layer "F.Cu") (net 17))
 (segment (start 112.8312 85.7054) (end 112.8312 82.0364) (width 0.5) (layer "F.Cu") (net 17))
 (segment (start 115.0152 85.8464) (end 112.9722 85.8464) (width 0.5) (layer "F.Cu") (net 17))
 (segment (start 112.7252 95.3628) (end 112.7252 93.98) (width 0.5) (layer "F.Cu") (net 17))
 (segment (start 112.8312 82.0364) (end 112.0552 81.2604) (width 0.5) (layer "F.Cu") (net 17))
 (segment (start 112.9722 85.8464) (end 112.8312 85.7054) (width 0.5) (layer "F.Cu") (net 17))
 (via (at 112.7252 93.98) (size 0.8) (drill 0.5) (layers "F.Cu" "B.Cu") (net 17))
 (via (at 112.8268 85.852) (size 0.8) (drill 0.5) (layers "F.Cu" "B.Cu") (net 17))
 (segment (start 112.7252 85.9536) (end 112.8268 85.852) (width 0.5) (layer "B.Cu") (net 17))
 (segment (start 112.7252 93.98) (end 112.7252 85.9536) (width 0.5) (layer "B.Cu") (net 17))
 (segment (start 111.1108 95.3628) (end 110.8456 95.3628) (width 0.5) (layer "F.Cu") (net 18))
 (segment (start 112.5108 96.7628) (end 111.1108 95.3628) (width 0.5) (layer "F.Cu") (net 18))
 (segment (start 112.7252 96.7628) (end 112.5108 96.7628) (width 0.5) (layer "F.Cu") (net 18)))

